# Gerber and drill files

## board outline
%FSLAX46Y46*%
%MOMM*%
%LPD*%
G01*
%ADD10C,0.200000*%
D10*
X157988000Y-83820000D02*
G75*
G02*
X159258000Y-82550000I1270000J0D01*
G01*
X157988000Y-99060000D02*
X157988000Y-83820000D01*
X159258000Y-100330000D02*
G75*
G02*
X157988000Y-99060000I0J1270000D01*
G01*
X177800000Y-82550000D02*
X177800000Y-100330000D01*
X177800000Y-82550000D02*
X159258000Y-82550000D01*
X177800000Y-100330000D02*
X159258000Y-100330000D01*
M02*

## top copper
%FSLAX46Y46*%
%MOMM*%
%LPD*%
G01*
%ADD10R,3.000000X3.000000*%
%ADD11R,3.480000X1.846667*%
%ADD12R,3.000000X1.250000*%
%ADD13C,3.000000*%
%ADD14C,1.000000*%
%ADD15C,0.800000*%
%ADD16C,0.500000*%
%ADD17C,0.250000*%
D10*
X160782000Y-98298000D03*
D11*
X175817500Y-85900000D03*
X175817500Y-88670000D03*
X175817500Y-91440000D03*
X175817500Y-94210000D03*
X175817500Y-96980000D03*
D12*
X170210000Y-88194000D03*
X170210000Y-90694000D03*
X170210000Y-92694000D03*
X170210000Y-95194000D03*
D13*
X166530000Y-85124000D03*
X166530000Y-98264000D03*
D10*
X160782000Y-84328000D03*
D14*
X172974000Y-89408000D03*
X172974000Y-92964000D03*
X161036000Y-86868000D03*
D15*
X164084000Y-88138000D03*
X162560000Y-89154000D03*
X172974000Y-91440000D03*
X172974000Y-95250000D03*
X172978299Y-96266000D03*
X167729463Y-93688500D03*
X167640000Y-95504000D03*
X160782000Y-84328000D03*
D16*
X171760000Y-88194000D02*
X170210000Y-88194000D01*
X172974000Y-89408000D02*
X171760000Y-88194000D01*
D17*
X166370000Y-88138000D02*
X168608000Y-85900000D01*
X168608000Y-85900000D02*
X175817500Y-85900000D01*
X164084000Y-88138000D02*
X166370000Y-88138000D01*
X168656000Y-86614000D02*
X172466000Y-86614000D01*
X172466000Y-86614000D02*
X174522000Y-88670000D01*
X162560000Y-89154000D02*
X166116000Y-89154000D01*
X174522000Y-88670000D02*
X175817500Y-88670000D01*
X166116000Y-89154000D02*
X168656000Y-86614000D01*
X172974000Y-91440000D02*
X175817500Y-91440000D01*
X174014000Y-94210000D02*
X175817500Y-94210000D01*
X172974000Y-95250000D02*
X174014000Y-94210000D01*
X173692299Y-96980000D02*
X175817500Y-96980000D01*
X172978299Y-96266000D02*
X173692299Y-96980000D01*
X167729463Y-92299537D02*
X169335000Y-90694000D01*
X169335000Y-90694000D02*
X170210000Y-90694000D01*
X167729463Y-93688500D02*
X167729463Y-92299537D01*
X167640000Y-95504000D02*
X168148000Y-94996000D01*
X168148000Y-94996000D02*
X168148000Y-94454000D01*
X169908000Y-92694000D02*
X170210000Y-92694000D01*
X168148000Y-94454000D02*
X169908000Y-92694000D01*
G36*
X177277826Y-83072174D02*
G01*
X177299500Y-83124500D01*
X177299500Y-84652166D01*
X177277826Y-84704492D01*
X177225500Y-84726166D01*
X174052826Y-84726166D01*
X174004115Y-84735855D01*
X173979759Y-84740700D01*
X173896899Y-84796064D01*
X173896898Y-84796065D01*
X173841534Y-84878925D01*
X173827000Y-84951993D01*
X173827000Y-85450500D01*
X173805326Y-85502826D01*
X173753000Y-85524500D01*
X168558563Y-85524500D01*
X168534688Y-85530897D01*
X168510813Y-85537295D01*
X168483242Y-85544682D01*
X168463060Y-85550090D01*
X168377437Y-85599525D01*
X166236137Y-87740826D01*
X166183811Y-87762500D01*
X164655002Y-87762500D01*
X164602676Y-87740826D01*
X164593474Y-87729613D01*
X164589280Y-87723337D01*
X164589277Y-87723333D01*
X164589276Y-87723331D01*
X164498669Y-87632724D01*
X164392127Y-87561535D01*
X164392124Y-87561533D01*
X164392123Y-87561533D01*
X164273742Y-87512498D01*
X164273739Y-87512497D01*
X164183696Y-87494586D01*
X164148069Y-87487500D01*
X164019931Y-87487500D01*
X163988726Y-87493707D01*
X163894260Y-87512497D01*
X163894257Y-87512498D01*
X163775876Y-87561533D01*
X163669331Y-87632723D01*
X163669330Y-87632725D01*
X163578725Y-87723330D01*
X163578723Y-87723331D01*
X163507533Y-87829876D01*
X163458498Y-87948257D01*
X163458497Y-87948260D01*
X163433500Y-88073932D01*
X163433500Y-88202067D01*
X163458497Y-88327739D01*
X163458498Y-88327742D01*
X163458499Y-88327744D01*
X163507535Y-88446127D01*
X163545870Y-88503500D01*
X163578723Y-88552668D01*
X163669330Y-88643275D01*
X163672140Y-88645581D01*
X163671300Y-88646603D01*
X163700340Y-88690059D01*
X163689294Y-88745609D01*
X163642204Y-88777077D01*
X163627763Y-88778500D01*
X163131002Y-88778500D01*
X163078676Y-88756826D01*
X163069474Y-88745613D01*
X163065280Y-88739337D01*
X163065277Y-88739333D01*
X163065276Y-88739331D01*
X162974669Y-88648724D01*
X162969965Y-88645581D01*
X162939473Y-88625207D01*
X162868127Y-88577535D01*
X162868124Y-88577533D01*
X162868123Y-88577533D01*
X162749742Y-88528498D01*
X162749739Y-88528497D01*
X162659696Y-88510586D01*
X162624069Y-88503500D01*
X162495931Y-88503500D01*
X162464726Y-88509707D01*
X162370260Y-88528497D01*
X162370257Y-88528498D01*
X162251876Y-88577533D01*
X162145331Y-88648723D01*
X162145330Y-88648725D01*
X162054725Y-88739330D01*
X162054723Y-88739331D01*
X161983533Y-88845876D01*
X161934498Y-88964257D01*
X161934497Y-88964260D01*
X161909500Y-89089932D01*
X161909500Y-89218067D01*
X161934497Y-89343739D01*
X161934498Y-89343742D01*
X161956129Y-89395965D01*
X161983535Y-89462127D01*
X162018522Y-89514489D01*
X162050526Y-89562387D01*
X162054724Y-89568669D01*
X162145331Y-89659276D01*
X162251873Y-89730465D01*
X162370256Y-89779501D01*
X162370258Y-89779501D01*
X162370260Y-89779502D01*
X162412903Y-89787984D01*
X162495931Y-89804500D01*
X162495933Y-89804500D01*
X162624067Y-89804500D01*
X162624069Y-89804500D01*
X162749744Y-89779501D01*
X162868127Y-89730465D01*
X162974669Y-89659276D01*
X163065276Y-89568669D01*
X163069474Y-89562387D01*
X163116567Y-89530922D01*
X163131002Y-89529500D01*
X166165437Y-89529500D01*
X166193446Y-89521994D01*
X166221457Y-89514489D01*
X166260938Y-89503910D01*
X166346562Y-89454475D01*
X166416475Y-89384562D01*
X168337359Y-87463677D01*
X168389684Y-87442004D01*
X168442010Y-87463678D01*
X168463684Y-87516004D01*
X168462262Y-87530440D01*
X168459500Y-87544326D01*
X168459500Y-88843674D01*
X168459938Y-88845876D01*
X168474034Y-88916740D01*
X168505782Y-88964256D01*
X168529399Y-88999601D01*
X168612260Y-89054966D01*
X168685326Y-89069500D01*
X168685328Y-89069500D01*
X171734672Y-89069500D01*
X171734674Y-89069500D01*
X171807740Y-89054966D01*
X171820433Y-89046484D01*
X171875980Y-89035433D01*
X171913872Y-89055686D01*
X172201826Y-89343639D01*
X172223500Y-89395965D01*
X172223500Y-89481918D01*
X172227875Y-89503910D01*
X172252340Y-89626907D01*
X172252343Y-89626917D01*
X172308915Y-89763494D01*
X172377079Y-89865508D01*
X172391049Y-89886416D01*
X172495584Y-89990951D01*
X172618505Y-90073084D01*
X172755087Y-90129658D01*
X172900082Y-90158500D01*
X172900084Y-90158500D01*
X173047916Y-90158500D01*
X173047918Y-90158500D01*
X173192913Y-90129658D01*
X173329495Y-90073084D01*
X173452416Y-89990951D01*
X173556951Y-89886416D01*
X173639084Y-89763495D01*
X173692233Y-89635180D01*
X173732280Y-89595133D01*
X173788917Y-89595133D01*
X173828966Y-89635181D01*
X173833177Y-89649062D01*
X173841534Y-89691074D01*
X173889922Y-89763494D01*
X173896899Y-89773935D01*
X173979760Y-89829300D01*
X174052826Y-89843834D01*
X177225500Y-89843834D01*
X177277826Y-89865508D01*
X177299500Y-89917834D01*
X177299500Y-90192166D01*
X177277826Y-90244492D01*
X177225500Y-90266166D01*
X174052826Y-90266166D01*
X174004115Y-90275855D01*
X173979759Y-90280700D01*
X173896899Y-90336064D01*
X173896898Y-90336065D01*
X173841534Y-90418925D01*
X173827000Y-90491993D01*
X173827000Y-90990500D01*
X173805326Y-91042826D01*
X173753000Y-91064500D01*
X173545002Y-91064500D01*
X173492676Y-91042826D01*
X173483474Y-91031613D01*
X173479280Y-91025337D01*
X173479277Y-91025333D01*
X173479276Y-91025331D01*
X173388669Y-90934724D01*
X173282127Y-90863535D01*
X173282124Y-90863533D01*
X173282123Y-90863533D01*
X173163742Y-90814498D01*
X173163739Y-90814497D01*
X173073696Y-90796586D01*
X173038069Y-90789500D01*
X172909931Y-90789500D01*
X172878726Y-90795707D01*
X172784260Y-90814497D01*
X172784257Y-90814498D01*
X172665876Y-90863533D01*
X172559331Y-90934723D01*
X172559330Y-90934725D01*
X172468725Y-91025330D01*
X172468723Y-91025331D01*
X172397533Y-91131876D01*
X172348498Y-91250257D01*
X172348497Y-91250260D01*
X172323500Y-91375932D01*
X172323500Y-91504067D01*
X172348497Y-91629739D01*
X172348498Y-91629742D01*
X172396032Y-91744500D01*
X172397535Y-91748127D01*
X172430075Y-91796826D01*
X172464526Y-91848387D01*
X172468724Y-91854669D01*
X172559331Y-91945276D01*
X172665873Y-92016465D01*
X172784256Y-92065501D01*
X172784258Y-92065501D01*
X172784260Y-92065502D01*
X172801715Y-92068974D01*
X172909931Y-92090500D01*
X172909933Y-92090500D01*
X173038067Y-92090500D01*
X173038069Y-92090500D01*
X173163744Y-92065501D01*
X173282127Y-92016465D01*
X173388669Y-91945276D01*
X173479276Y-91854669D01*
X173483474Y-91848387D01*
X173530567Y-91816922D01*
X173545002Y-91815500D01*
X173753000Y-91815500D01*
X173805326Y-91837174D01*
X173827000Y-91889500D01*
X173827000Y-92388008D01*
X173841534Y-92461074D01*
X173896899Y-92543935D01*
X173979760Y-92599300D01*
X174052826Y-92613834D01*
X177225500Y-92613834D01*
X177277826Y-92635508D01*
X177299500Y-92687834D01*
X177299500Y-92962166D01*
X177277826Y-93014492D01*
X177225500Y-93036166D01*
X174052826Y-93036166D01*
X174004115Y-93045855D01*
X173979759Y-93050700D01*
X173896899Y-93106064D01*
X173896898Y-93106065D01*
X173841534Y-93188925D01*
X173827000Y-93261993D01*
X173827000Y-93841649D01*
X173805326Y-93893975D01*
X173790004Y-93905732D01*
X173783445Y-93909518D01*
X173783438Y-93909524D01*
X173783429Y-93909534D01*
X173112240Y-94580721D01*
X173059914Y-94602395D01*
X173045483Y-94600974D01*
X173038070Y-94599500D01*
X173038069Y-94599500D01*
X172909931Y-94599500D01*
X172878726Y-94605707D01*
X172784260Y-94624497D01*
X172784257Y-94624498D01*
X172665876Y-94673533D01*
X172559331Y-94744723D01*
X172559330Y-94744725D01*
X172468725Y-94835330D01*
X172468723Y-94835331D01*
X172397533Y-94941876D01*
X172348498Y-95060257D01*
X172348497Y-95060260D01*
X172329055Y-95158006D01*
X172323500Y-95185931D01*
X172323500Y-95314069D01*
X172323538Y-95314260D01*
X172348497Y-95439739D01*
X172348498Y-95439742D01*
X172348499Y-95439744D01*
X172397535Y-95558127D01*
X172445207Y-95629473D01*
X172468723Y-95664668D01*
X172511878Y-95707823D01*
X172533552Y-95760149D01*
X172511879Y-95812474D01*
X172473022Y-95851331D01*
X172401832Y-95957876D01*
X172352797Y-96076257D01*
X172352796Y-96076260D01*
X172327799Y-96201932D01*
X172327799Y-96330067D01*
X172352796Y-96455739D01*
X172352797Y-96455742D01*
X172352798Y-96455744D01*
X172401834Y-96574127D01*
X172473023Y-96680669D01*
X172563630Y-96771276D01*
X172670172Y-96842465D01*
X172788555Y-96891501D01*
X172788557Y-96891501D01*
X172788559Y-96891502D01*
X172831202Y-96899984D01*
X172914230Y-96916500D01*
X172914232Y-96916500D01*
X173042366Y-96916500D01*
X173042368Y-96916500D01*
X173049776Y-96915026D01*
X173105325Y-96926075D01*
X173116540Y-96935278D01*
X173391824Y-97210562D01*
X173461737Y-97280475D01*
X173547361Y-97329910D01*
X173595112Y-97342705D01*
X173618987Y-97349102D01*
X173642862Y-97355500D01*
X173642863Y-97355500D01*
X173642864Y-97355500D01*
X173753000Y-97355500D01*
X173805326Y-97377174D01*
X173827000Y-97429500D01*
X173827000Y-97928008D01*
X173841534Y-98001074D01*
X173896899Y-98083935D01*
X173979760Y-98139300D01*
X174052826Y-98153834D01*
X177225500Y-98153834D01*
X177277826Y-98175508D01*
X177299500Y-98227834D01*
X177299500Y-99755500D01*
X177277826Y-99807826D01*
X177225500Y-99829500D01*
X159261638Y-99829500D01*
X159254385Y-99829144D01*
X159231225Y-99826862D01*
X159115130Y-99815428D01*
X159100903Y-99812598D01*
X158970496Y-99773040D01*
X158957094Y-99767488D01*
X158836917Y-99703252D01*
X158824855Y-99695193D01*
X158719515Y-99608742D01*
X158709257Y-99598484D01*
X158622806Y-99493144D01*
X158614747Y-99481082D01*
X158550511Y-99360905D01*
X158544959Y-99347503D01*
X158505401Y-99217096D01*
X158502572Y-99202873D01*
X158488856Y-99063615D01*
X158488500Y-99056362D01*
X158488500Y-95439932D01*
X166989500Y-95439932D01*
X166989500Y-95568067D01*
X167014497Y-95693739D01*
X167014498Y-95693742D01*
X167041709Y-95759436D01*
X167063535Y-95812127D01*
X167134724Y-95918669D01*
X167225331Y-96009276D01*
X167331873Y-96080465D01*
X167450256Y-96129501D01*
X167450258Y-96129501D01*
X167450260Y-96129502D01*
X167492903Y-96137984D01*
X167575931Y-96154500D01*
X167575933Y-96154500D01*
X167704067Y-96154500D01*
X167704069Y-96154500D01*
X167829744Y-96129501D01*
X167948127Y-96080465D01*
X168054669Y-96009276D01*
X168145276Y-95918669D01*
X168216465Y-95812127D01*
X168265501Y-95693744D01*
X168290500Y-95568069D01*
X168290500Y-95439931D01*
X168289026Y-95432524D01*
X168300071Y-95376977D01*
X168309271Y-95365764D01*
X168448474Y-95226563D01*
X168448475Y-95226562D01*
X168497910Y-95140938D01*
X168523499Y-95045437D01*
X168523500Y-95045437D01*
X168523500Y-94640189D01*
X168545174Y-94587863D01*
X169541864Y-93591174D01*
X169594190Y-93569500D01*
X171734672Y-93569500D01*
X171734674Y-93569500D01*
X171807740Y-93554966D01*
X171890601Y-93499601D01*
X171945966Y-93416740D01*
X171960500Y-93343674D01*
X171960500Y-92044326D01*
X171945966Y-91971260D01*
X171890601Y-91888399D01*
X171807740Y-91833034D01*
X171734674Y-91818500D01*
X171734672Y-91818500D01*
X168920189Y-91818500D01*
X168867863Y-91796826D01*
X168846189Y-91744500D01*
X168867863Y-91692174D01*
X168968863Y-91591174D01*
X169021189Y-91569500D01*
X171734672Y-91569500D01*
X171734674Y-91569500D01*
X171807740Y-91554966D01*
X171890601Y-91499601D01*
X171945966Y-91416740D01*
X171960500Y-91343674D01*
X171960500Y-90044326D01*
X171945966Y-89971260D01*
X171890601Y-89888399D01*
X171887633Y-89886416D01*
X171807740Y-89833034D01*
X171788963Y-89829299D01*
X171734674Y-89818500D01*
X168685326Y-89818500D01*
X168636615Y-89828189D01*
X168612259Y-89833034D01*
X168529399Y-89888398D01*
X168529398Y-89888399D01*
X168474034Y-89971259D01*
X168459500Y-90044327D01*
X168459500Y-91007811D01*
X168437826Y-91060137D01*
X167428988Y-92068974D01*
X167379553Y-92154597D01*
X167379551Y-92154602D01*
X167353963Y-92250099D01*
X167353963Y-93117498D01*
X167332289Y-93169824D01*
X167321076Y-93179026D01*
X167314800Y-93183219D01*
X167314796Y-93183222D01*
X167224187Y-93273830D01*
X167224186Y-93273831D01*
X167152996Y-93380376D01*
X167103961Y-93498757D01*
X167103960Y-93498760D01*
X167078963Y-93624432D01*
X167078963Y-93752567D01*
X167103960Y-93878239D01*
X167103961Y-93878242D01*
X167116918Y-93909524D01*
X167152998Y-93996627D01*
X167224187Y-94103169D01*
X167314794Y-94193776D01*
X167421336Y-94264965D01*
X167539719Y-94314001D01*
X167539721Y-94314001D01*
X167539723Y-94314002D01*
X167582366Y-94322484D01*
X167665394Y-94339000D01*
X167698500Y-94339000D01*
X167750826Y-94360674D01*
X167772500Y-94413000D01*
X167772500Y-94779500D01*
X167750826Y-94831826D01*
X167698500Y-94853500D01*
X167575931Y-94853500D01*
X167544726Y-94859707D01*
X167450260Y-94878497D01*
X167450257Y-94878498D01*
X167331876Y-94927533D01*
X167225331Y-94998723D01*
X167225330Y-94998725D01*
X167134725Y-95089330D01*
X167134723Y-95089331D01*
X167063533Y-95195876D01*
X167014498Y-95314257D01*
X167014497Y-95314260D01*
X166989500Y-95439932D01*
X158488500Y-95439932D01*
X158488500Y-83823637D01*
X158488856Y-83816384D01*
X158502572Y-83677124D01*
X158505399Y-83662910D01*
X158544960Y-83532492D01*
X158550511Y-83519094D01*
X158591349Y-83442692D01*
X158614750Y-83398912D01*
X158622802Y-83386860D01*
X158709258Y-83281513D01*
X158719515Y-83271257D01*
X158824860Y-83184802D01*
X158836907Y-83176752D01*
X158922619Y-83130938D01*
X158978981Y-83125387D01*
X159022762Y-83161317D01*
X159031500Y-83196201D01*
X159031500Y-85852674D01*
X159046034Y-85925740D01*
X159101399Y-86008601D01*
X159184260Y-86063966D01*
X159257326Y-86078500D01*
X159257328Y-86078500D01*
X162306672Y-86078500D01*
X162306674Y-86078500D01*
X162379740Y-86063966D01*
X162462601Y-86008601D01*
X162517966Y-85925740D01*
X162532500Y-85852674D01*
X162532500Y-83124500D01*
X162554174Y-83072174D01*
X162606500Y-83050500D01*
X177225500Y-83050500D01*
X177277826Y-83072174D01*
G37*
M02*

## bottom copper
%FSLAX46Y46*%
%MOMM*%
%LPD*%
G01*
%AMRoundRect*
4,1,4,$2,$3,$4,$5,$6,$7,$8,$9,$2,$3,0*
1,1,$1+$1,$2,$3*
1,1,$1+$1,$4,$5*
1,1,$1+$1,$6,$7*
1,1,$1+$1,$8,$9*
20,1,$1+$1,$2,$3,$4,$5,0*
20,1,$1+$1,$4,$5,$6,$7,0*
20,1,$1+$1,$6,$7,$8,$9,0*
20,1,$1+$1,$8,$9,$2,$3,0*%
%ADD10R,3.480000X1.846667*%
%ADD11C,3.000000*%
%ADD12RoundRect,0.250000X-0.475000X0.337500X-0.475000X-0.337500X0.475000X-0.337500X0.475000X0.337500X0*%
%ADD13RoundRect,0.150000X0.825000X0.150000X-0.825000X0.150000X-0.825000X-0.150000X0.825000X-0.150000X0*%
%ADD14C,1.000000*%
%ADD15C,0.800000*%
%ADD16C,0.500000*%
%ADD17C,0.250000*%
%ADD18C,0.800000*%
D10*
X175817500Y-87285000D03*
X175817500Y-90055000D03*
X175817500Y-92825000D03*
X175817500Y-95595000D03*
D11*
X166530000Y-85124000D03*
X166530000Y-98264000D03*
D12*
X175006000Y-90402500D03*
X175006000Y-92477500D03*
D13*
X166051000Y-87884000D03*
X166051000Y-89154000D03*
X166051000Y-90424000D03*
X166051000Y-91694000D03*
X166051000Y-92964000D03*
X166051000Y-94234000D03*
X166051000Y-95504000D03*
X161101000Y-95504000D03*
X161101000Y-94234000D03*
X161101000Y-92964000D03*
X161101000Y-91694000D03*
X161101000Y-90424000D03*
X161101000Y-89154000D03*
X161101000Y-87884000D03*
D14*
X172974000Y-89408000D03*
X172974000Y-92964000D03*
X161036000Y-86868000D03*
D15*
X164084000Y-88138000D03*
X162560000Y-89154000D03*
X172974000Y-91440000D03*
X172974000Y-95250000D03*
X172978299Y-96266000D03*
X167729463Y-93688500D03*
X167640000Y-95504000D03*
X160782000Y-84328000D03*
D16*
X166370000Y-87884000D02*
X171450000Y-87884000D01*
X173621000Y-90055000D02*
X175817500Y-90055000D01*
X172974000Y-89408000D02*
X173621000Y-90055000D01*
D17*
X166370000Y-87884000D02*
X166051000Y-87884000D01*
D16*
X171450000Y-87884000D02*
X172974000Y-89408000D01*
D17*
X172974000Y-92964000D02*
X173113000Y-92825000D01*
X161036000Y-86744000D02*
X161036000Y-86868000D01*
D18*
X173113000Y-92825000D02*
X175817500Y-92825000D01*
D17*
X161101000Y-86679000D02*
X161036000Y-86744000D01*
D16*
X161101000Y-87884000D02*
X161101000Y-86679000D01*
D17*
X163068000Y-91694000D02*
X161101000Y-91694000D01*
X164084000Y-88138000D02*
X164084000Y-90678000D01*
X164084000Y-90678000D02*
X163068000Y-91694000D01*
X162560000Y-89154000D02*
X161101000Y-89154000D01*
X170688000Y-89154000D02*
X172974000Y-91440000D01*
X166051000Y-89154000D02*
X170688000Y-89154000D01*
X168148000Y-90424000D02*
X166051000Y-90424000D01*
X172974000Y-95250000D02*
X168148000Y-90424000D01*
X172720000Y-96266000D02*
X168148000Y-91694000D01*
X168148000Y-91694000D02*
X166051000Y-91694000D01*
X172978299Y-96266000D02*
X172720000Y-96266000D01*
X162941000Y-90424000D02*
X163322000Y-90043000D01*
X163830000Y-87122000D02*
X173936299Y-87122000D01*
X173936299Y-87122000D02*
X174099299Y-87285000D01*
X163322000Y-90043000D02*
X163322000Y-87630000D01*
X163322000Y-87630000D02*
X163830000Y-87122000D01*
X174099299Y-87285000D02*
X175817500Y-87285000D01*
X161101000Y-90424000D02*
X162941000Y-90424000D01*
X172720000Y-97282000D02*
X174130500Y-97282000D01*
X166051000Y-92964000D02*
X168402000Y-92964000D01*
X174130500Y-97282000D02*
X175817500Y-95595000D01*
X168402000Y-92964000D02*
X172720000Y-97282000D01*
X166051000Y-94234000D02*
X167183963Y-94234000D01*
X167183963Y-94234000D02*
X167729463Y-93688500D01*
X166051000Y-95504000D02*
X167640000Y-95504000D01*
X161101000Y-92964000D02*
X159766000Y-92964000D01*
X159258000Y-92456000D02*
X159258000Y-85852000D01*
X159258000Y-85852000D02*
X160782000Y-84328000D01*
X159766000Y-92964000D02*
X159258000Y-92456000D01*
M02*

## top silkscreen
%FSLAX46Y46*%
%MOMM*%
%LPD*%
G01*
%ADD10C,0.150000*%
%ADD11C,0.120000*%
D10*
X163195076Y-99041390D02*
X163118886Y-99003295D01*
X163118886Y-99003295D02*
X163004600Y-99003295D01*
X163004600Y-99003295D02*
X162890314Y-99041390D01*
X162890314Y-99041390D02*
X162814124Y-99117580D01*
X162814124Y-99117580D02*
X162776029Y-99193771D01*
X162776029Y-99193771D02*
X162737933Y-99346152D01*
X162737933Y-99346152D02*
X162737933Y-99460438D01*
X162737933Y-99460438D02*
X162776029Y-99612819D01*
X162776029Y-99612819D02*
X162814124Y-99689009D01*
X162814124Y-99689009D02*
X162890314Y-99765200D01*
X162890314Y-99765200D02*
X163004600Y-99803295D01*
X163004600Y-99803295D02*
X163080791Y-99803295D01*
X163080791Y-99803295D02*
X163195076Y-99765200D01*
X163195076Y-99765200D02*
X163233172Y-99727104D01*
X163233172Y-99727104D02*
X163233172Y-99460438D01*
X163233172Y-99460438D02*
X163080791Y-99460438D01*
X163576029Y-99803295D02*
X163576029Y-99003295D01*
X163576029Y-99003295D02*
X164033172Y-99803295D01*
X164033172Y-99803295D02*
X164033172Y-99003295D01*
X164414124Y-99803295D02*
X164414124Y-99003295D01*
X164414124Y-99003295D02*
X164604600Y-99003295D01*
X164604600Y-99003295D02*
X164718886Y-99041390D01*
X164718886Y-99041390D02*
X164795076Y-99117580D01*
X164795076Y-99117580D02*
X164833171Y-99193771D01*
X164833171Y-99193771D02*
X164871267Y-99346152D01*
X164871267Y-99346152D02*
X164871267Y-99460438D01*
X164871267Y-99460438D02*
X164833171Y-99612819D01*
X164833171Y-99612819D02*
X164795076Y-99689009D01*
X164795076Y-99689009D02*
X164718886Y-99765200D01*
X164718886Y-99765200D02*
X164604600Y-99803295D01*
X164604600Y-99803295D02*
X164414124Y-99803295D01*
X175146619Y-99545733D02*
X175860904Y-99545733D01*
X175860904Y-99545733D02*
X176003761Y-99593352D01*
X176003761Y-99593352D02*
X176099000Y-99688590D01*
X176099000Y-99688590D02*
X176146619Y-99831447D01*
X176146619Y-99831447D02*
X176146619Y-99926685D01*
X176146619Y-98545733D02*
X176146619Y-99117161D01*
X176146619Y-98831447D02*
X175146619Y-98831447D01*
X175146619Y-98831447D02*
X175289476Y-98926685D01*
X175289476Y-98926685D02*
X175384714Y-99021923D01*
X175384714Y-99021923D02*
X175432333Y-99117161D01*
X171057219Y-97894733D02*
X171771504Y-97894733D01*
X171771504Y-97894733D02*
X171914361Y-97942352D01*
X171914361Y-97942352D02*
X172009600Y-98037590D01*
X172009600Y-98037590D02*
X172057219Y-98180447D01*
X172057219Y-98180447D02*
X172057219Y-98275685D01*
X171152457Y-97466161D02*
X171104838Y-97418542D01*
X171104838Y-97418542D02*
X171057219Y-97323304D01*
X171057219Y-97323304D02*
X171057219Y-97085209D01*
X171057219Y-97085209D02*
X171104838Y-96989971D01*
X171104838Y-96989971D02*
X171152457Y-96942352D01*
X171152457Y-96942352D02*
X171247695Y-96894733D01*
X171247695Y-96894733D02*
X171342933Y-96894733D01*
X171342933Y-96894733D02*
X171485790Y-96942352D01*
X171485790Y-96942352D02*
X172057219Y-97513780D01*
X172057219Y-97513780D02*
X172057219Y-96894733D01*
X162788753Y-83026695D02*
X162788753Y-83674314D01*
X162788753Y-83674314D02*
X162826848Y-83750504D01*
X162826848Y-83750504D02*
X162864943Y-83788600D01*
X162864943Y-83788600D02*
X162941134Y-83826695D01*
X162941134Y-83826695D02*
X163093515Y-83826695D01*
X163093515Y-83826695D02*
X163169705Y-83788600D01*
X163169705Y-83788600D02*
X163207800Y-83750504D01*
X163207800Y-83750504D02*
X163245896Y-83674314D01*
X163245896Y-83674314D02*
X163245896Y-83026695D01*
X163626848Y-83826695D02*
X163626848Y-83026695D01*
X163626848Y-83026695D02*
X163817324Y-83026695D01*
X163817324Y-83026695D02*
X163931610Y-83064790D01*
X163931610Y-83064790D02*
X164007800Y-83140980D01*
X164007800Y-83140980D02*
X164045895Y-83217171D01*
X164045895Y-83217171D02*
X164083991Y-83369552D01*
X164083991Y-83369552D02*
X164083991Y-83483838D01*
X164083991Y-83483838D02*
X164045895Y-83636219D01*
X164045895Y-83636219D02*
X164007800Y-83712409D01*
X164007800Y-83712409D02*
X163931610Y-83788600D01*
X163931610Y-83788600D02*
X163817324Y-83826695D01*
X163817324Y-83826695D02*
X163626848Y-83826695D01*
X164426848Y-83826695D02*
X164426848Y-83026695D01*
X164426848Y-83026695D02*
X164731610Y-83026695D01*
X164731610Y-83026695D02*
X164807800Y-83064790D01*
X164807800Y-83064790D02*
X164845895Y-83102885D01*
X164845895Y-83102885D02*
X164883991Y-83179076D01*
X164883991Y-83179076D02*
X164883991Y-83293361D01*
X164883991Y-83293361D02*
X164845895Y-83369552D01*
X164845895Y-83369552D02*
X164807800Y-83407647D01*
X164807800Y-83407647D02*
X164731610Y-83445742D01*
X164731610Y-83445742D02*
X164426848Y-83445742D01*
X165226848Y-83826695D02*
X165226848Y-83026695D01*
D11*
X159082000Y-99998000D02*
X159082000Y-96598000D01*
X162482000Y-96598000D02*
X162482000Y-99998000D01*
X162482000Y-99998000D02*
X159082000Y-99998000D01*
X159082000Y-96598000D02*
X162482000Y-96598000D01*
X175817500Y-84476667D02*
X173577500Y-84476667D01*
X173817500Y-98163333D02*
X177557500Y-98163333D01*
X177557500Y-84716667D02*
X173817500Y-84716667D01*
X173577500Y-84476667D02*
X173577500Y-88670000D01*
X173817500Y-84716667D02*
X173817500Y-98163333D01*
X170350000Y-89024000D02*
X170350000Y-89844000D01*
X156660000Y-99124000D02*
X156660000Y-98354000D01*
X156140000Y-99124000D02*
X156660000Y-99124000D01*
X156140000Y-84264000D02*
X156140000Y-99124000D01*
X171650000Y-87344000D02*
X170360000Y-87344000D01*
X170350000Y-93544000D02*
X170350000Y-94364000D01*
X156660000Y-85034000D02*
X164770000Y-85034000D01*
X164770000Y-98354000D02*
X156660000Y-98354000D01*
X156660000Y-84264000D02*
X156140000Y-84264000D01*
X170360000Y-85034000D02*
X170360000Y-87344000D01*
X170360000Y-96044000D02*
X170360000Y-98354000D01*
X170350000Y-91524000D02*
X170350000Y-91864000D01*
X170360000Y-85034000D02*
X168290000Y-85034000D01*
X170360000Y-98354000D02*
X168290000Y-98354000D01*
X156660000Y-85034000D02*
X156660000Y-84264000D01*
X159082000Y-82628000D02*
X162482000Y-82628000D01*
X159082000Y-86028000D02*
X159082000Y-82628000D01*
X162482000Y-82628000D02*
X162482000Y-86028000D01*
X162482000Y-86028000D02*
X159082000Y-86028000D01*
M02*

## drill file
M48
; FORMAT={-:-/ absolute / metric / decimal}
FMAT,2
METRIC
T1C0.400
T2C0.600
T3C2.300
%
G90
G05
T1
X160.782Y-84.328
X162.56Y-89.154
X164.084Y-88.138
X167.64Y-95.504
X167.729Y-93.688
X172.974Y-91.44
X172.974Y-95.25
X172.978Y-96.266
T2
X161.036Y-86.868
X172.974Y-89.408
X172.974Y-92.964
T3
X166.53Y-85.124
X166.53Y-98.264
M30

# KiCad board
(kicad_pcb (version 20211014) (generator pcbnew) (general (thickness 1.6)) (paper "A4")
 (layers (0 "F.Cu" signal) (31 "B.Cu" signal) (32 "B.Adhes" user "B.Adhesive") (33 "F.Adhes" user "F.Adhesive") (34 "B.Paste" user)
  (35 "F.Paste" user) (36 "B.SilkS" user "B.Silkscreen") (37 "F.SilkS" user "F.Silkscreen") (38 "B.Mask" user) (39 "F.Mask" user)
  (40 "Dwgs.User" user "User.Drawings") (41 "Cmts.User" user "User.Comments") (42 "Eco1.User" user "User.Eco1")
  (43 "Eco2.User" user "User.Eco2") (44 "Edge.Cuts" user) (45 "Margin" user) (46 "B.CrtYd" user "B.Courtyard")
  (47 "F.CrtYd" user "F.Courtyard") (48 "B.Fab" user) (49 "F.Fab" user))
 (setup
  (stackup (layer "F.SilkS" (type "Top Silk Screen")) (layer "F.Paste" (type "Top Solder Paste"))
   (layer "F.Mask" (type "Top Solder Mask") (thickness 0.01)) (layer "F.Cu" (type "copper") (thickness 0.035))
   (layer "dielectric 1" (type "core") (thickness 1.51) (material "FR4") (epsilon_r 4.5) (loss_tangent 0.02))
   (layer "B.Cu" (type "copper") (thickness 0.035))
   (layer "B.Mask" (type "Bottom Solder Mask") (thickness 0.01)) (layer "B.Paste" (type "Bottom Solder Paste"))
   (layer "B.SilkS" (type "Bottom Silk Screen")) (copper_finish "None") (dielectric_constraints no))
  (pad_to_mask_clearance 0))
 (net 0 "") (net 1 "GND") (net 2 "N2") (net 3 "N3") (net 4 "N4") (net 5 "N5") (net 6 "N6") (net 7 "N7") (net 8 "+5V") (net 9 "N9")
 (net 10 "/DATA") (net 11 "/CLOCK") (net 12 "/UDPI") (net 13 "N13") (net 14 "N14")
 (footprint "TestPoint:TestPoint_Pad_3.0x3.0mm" (layer "F.Cu") (at 160.782 98.298)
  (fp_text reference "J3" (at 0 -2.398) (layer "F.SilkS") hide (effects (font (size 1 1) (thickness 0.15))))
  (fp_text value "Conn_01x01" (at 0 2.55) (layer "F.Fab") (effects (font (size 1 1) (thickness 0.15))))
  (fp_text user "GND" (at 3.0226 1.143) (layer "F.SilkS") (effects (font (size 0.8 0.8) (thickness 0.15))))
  (fp_line (start -1.7 1.7) (end -1.7 -1.7) (layer "F.SilkS") (width 0.12))
  (fp_line (start 1.7 -1.7) (end 1.7 1.7) (layer "F.SilkS") (width 0.12))
  (fp_line (start 1.7 1.7) (end -1.7 1.7) (layer "F.SilkS") (width 0.12))
  (fp_line (start -1.7 -1.7) (end 1.7 -1.7) (layer "F.SilkS") (width 0.12))
  (pad "1" smd rect (at 0 0) (size 3 3) (layers "F.Cu" "F.Mask") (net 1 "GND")))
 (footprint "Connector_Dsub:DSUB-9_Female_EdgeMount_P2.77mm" (layer "F.Cu") (at 175.8175 91.44 90)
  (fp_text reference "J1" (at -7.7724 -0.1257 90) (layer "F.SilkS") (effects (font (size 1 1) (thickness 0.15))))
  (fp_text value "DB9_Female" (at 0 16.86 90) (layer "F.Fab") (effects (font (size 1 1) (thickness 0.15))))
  (fp_line (start 6.963333 0) (end 6.963333 -2.24) (layer "F.SilkS") (width 0.12))
  (fp_line (start -6.723333 -2) (end -6.723333 1.74) (layer "F.SilkS") (width 0.12))
  (fp_line (start 6.723333 1.74) (end 6.723333 -2) (layer "F.SilkS") (width 0.12))
  (fp_line (start 6.963333 -2.24) (end 2.77 -2.24) (layer "F.SilkS") (width 0.12))
  (fp_line (start 6.723333 -2) (end -6.723333 -2) (layer "F.SilkS") (width 0.12))
  (pad "1" smd rect (at 5.54 0 90) (size 1.846667 3.48) (layers "F.Cu" "F.Paste" "F.Mask") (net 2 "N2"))
  (pad "2" smd rect (at 2.77 0 90) (size 1.846667 3.48) (layers "F.Cu" "F.Paste" "F.Mask") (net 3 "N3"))
  (pad "3" smd rect (at 0 0 90) (size 1.846667 3.48) (layers "F.Cu" "F.Paste" "F.Mask") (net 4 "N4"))
  (pad "4" smd rect (at -2.77 0 90) (size 1.846667 3.48) (layers "F.Cu" "F.Paste" "F.Mask") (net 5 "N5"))
  (pad "5" smd rect (at -5.54 0 90) (size 1.846667 3.48) (layers "F.Cu" "F.Paste" "F.Mask") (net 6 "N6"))
  (pad "6" smd rect (at 4.155 0 90) (size 1.846667 3.48) (layers "B.Cu" "B.Paste" "B.Mask") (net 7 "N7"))
  (pad "7" smd rect (at 1.385 0 90) (size 1.846667 3.48) (layers "B.Cu" "B.Paste" "B.Mask") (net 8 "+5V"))
  (pad "8" smd rect (at -1.385 0 90) (size 1.846667 3.48) (layers "B.Cu" "B.Paste" "B.Mask") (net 1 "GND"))
  (pad "9" smd rect (at -4.155 0 90) (size 1.846667 3.48) (layers "B.Cu" "B.Paste" "B.Mask") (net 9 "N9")))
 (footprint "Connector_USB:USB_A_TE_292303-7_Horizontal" (layer "F.Cu") (at 163.83 91.694 -90)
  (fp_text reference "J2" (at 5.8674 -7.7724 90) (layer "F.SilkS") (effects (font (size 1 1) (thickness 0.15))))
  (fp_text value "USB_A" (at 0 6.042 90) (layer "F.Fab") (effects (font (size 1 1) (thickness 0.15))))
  (fp_line (start -2.67 -6.52) (end -1.85 -6.52) (layer "F.SilkS") (width 0.12))
  (fp_line (start 7.43 7.17) (end 6.66 7.17) (layer "F.SilkS") (width 0.12))
  (fp_line (start 7.43 7.69) (end 7.43 7.17) (layer "F.SilkS") (width 0.12))
  (fp_line (start -7.43 7.69) (end 7.43 7.69) (layer "F.SilkS") (width 0.12))
  (fp_line (start -4.35 -7.82) (end -4.35 -6.53) (layer "F.SilkS") (width 0.12))
  (fp_line (start 1.85 -6.52) (end 2.67 -6.52) (layer "F.SilkS") (width 0.12))
  (fp_line (start -6.66 7.17) (end -6.66 -0.94) (layer "F.SilkS") (width 0.12))
  (fp_line (start 6.66 -0.94) (end 6.66 7.17) (layer "F.SilkS") (width 0.12))
  (fp_line (start -7.43 7.17) (end -7.43 7.69) (layer "F.SilkS") (width 0.12))
  (fp_line (start -6.66 -6.53) (end -4.35 -6.53) (layer "F.SilkS") (width 0.12))
  (fp_line (start 4.35 -6.53) (end 6.66 -6.53) (layer "F.SilkS") (width 0.12))
  (fp_line (start -0.17 -6.52) (end 0.17 -6.52) (layer "F.SilkS") (width 0.12))
  (fp_line (start -6.66 -6.53) (end -6.66 -4.46) (layer "F.SilkS") (width 0.12))
  (fp_line (start 6.66 -6.53) (end 6.66 -4.46) (layer "F.SilkS") (width 0.12))
  (fp_line (start -6.66 7.17) (end -7.43 7.17) (layer "F.SilkS") (width 0.12))
  (pad "1" smd rect (at -3.5 -6.38 270) (size 1.25 3) (layers "F.Cu" "F.Paste" "F.Mask") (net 8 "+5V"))
  (pad "2" smd rect (at -1 -6.38 270) (size 1.25 3) (layers "F.Cu" "F.Paste" "F.Mask") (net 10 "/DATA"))
  (pad "3" smd rect (at 1 -6.38 270) (size 1.25 3) (layers "F.Cu" "F.Paste" "F.Mask") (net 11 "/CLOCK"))
  (pad "4" smd rect (at 3.5 -6.38 270) (size 1.25 3) (layers "F.Cu" "F.Paste" "F.Mask") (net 1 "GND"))
  (pad "5" thru_hole circle (at -6.57 -2.7 270) (size 3 3) (drill 2.3) (layers *.Cu *.Mask) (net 1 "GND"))
  (pad "5" thru_hole circle (at 6.57 -2.7 270) (size 3 3) (drill 2.3) (layers *.Cu *.Mask) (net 1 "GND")))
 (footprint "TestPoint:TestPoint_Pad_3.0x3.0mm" (layer "F.Cu") (at 160.782 84.328)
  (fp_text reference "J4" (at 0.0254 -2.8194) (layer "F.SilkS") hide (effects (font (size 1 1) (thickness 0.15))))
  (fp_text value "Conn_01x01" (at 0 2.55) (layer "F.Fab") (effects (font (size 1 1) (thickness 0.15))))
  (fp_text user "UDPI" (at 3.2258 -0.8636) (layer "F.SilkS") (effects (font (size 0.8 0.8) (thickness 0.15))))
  (fp_line (start -1.7 -1.7) (end 1.7 -1.7) (layer "F.SilkS") (width 0.12))
  (fp_line (start -1.7 1.7) (end -1.7 -1.7) (layer "F.SilkS") (width 0.12))
  (fp_line (start 1.7 -1.7) (end 1.7 1.7) (layer "F.SilkS") (width 0.12))
  (fp_line (start 1.7 1.7) (end -1.7 1.7) (layer "F.SilkS") (width 0.12))
  (pad "1" smd rect (at 0 0) (size 3 3) (layers "F.Cu" "F.Mask") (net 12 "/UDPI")))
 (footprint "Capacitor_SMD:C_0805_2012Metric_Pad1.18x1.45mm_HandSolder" (layer "B.Cu") (at 175.006 91.44 -90)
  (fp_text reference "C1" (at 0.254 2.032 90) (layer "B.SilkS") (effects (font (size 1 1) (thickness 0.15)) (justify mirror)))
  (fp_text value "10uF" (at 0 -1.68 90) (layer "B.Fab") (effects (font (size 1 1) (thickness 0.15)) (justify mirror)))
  (pad "1" smd roundrect (at -1.0375 0 270) (size 1.175 1.45) (layers "B.Cu" "B.Paste" "B.Mask") (roundrect_rratio 0.2127659574)
   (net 8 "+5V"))
  (pad "2" smd roundrect (at 1.0375 0 270) (size 1.175 1.45) (layers "B.Cu" "B.Paste" "B.Mask") (roundrect_rratio 0.2127659574)
   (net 1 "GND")))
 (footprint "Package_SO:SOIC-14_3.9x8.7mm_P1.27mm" (layer "B.Cu") (at 163.576 91.694 180)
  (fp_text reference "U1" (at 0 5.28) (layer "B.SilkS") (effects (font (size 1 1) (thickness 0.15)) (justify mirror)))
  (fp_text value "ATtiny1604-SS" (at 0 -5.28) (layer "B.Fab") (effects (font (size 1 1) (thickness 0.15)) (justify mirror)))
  (pad "1" smd roundrect (at -2.475 3.81 180) (size 1.95 0.6) (layers "B.Cu" "B.Paste" "B.Mask") (roundrect_rratio 0.25) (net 8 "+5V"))
  (pad "2" smd roundrect (at -2.475 2.54 180) (size 1.95 0.6) (layers "B.Cu" "B.Paste" "B.Mask") (roundrect_rratio 0.25) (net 4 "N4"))
  (pad "3" smd roundrect (at -2.475 1.27 180) (size 1.95 0.6) (layers "B.Cu" "B.Paste" "B.Mask") (roundrect_rratio 0.25) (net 5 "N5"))
  (pad "4" smd roundrect (at -2.475 0 180) (size 1.95 0.6) (layers "B.Cu" "B.Paste" "B.Mask") (roundrect_rratio 0.25) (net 6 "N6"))
  (pad "5" smd roundrect (at -2.475 -1.27 180) (size 1.95 0.6) (layers "B.Cu" "B.Paste" "B.Mask") (roundrect_rratio 0.25) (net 9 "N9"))
  (pad "6" smd roundrect (at -2.475 -2.54 180) (size 1.95 0.6) (layers "B.Cu" "B.Paste" "B.Mask") (roundrect_rratio 0.25) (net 10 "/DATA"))
  (pad "7" smd roundrect (at -2.475 -3.81 180) (size 1.95 0.6) (layers "B.Cu" "B.Paste" "B.Mask") (roundrect_rratio 0.25) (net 11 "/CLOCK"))
  (pad "8" smd roundrect (at 2.475 -3.81 180) (size 1.95 0.6) (layers "B.Cu" "B.Paste" "B.Mask") (roundrect_rratio 0.25) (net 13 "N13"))
  (pad "9" smd roundrect (at 2.475 -2.54 180) (size 1.95 0.6) (layers "B.Cu" "B.Paste" "B.Mask") (roundrect_rratio 0.25) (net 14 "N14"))
  (pad "10" smd roundrect (at 2.475 -1.27 180) (size 1.95 0.6) (layers "B.Cu" "B.Paste" "B.Mask") (roundrect_rratio 0.25) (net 12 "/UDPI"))
  (pad "11" smd roundrect (at 2.475 0 180) (size 1.95 0.6) (layers "B.Cu" "B.Paste" "B.Mask") (roundrect_rratio 0.25) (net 2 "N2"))
  (pad "12" smd roundrect (at 2.475 1.27 180) (size 1.95 0.6) (layers "B.Cu" "B.Paste" "B.Mask") (roundrect_rratio 0.25) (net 7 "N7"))
  (pad "13" smd roundrect (at 2.475 2.54 180) (size 1.95 0.6) (layers "B.Cu" "B.Paste" "B.Mask") (roundrect_rratio 0.25) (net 3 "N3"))
  (pad "14" smd roundrect (at 2.475 3.81 180) (size 1.95 0.6) (layers "B.Cu" "B.Paste" "B.Mask") (roundrect_rratio 0.25) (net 1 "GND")))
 (gr_arc (start 157.988 83.82) (mid 158.359974 82.921974) (end 159.258 82.55) (layer "Edge.Cuts") (width 0.2))
 (gr_line (start 157.988 99.06) (end 157.988 83.82) (layer "Edge.Cuts") (width 0.2))
 (gr_arc (start 159.258 100.33) (mid 158.359974 99.958026) (end 157.988 99.06) (layer "Edge.Cuts") (width 0.2))
 (gr_line (start 177.8 82.55) (end 177.8 100.33) (layer "Edge.Cuts") (width 0.2))
 (gr_line (start 177.8 82.55) (end 159.258 82.55) (layer "Edge.Cuts") (width 0.2))
 (gr_line (start 177.8 100.33) (end 159.258 100.33) (layer "Edge.Cuts") (width 0.2))
 (segment (start 171.76 88.194) (end 170.21 88.194) (width 0.5) (layer "F.Cu") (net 8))
 (segment (start 172.974 89.408) (end 171.76 88.194) (width 0.5) (layer "F.Cu") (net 8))
 (via (at 172.974 89.408) (size 1) (drill 0.6) (layers "F.Cu" "B.Cu") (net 8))
 (segment (start 166.37 87.884) (end 171.45 87.884) (width 0.5) (layer "B.Cu") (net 8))
 (segment (start 173.621 90.055) (end 175.8175 90.055) (width 0.5) (layer "B.Cu") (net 8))
 (segment (start 172.974 89.408) (end 173.621 90.055) (width 0.5) (layer "B.Cu") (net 8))
 (segment (start 166.37 87.884) (end 166.051 87.884) (width 0.25) (layer "B.Cu") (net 8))
 (segment (start 171.45 87.884) (end 172.974 89.408) (width 0.5) (layer "B.Cu") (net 8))
 (via (at 172.974 92.964) (size 1) (drill 0.6) (layers "F.Cu" "B.Cu") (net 1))
 (via (at 161.036 86.868) (size 1) (drill 0.6) (layers "F.Cu" "B.Cu") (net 1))
 (segment (start 172.974 92.964) (end 173.113 92.825) (width 0.25) (layer "B.Cu") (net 1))
 (segment (start 161.036 86.744) (end 161.036 86.868) (width 0.25) (layer "B.Cu") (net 1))
 (segment (start 173.113 92.825) (end 175.8175 92.825) (width 0.8) (layer "B.Cu") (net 1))
 (segment (start 161.101 86.679) (end 161.036 86.744) (width 0.25) (layer "B.Cu") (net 1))
 (segment (start 161.101 87.884) (end 161.101 86.679) (width 0.5) (layer "B.Cu") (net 1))
 (segment (start 166.37 88.138) (end 168.608 85.9) (width 0.25) (layer "F.Cu") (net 2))
 (segment (start 168.608 85.9) (end 175.8175 85.9) (width 0.25) (layer "F.Cu") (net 2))
 (segment (start 164.084 88.138) (end 166.37 88.138) (width 0.25) (layer "F.Cu") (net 2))
 (via (at 164.084 88.138) (size 0.8) (drill 0.4) (layers "F.Cu" "B.Cu") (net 2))
 (segment (start 163.068 91.694) (end 161.101 91.694) (width 0.25) (layer "B.Cu") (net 2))
 (segment (start 164.084 88.138) (end 164.084 90.678) (width 0.25) (layer "B.Cu") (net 2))
 (segment (start 164.084 90.678) (end 163.068 91.694) (width 0.25) (layer "B.Cu") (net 2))
 (segment (start 168.656 86.614) (end 172.466 86.614) (width 0.25) (layer "F.Cu") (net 3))
 (segment (start 172.466 86.614) (end 174.522 88.67) (width 0.25) (layer "F.Cu") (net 3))
 (segment (start 162.56 89.154) (end 166.116 89.154) (width 0.25) (layer "F.Cu") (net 3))
 (segment (start 174.522 88.67) (end 175.8175 88.67) (width 0.25) (layer "F.Cu") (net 3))
 (segment (start 166.116 89.154) (end 168.656 86.614) (width 0.25) (layer "F.Cu") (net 3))
 (via (at 162.56 89.154) (size 0.8) (drill 0.4) (layers "F.Cu" "B.Cu") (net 3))
 (segment (start 162.56 89.154) (end 161.101 89.154) (width 0.25) (layer "B.Cu") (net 3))
 (segment (start 172.974 91.44) (end 175.8175 91.44) (width 0.25) (layer "F.Cu") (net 4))
 (via (at 172.974 91.44) (size 0.8) (drill 0.4) (layers "F.Cu" "B.Cu") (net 4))
 (segment (start 170.688 89.154) (end 172.974 91.44) (width 0.25) (layer "B.Cu") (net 4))
 (segment (start 166.051 89.154) (end 170.688 89.154) (width 0.25) (layer "B.Cu") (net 4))
 (segment (start 174.014 94.21) (end 175.8175 94.21) (width 0.25) (layer "F.Cu") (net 5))
 (segment (start 172.974 95.25) (end 174.014 94.21) (width 0.25) (layer "F.Cu") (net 5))
 (via (at 172.974 95.25) (size 0.8) (drill 0.4) (layers "F.Cu" "B.Cu") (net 5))
 (segment (start 168.148 90.424) (end 166.051 90.424) (width 0.25) (layer "B.Cu") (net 5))
 (segment (start 172.974 95.25) (end 168.148 90.424) (width 0.25) (layer "B.Cu") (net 5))
 (segment (start 173.692299 96.98) (end 175.8175 96.98) (width 0.25) (layer "F.Cu") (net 6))
 (segment (start 172.978299 96.266) (end 173.692299 96.98) (width 0.25) (layer "F.Cu") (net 6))
 (via (at 172.978299 96.266) (size 0.8) (drill 0.4) (layers "F.Cu" "B.Cu") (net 6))
 (segment (start 172.72 96.266) (end 168.148 91.694) (width 0.25) (layer "B.Cu") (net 6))
 (segment (start 168.148 91.694) (end 166.051 91.694) (width 0.25) (layer "B.Cu") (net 6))
 (segment (start 172.978299 96.266) (end 172.72 96.266) (width 0.25) (layer "B.Cu") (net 6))
 (segment (start 162.941 90.424) (end 163.322 90.043) (width 0.25) (layer "B.Cu") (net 7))
 (segment (start 163.83 87.122) (end 173.936299 87.122) (width 0.25) (layer "B.Cu") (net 7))
 (segment (start 173.936299 87.122) (end 174.099299 87.285) (width 0.25) (layer "B.Cu") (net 7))
 (segment (start 163.322 90.043) (end 163.322 87.63) (width 0.25) (layer "B.Cu") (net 7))
 (segment (start 163.322 87.63) (end 163.83 87.122) (width 0.25) (layer "B.Cu") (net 7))
 (segment (start 174.099299 87.285) (end 175.8175 87.285) (width 0.25) (layer "B.Cu") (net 7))
 (segment (start 161.101 90.424) (end 162.941 90.424) (width 0.25) (layer "B.Cu") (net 7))
 (segment (start 172.72 97.282) (end 174.1305 97.282) (width 0.25) (layer "B.Cu") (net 9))
 (segment (start 166.051 92.964) (end 168.402 92.964) (width 0.25) (layer "B.Cu") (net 9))
 (segment (start 174.1305 97.282) (end 175.8175 95.595) (width 0.25) (layer "B.Cu") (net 9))
 (segment (start 168.402 92.964) (end 172.72 97.282) (width 0.25) (layer "B.Cu") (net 9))
 (segment (start 167.729463 92.299537) (end 169.335 90.694) (width 0.25) (layer "F.Cu") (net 10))
 (segment (start 169.335 90.694) (end 170.21 90.694) (width 0.25) (layer "F.Cu") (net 10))
 (segment (start 167.729463 93.6885) (end 167.729463 92.299537) (width 0.25) (layer "F.Cu") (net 10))
 (via (at 167.729463 93.6885) (size 0.8) (drill 0.4) (layers "F.Cu" "B.Cu") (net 10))
 (segment (start 166.051 94.234) (end 167.183963 94.234) (width 0.25) (layer "B.Cu") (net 10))
 (segment (start 167.183963 94.234) (end 167.729463 93.6885) (width 0.25) (layer "B.Cu") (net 10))
 (segment (start 167.64 95.504) (end 168.148 94.996) (width 0.25) (layer "F.Cu") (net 11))
 (segment (start 168.148 94.996) (end 168.148 94.454) (width 0.25) (layer "F.Cu") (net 11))
 (segment (start 169.908 92.694) (end 170.21 92.694) (width 0.25) (layer "F.Cu") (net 11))
 (segment (start 168.148 94.454) (end 169.908 92.694) (width 0.25) (layer "F.Cu") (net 11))
 (via (at 167.64 95.504) (size 0.8) (drill 0.4) (layers "F.Cu" "B.Cu") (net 11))
 (segment (start 166.051 95.504) (end 167.64 95.504) (width 0.25) (layer "B.Cu") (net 11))
 (via (at 160.782 84.328) (size 0.8) (drill 0.4) (layers "F.Cu" "B.Cu") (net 12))
 (segment (start 161.101 92.964) (end 159.766 92.964) (width 0.25) (layer "B.Cu") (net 12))
 (segment (start 159.258 92.456) (end 159.258 85.852) (width 0.25) (layer "B.Cu") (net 12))
 (segment (start 159.258 85.852) (end 160.782 84.328) (width 0.25) (layer "B.Cu") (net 12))
 (segment (start 159.766 92.964) (end 159.258 92.456) (width 0.25) (layer "B.Cu") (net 12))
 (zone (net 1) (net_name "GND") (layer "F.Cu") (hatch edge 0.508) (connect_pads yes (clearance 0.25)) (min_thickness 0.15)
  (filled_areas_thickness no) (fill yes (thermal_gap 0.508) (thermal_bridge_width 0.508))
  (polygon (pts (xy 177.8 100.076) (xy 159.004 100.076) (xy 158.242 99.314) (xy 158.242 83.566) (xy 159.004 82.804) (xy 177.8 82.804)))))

